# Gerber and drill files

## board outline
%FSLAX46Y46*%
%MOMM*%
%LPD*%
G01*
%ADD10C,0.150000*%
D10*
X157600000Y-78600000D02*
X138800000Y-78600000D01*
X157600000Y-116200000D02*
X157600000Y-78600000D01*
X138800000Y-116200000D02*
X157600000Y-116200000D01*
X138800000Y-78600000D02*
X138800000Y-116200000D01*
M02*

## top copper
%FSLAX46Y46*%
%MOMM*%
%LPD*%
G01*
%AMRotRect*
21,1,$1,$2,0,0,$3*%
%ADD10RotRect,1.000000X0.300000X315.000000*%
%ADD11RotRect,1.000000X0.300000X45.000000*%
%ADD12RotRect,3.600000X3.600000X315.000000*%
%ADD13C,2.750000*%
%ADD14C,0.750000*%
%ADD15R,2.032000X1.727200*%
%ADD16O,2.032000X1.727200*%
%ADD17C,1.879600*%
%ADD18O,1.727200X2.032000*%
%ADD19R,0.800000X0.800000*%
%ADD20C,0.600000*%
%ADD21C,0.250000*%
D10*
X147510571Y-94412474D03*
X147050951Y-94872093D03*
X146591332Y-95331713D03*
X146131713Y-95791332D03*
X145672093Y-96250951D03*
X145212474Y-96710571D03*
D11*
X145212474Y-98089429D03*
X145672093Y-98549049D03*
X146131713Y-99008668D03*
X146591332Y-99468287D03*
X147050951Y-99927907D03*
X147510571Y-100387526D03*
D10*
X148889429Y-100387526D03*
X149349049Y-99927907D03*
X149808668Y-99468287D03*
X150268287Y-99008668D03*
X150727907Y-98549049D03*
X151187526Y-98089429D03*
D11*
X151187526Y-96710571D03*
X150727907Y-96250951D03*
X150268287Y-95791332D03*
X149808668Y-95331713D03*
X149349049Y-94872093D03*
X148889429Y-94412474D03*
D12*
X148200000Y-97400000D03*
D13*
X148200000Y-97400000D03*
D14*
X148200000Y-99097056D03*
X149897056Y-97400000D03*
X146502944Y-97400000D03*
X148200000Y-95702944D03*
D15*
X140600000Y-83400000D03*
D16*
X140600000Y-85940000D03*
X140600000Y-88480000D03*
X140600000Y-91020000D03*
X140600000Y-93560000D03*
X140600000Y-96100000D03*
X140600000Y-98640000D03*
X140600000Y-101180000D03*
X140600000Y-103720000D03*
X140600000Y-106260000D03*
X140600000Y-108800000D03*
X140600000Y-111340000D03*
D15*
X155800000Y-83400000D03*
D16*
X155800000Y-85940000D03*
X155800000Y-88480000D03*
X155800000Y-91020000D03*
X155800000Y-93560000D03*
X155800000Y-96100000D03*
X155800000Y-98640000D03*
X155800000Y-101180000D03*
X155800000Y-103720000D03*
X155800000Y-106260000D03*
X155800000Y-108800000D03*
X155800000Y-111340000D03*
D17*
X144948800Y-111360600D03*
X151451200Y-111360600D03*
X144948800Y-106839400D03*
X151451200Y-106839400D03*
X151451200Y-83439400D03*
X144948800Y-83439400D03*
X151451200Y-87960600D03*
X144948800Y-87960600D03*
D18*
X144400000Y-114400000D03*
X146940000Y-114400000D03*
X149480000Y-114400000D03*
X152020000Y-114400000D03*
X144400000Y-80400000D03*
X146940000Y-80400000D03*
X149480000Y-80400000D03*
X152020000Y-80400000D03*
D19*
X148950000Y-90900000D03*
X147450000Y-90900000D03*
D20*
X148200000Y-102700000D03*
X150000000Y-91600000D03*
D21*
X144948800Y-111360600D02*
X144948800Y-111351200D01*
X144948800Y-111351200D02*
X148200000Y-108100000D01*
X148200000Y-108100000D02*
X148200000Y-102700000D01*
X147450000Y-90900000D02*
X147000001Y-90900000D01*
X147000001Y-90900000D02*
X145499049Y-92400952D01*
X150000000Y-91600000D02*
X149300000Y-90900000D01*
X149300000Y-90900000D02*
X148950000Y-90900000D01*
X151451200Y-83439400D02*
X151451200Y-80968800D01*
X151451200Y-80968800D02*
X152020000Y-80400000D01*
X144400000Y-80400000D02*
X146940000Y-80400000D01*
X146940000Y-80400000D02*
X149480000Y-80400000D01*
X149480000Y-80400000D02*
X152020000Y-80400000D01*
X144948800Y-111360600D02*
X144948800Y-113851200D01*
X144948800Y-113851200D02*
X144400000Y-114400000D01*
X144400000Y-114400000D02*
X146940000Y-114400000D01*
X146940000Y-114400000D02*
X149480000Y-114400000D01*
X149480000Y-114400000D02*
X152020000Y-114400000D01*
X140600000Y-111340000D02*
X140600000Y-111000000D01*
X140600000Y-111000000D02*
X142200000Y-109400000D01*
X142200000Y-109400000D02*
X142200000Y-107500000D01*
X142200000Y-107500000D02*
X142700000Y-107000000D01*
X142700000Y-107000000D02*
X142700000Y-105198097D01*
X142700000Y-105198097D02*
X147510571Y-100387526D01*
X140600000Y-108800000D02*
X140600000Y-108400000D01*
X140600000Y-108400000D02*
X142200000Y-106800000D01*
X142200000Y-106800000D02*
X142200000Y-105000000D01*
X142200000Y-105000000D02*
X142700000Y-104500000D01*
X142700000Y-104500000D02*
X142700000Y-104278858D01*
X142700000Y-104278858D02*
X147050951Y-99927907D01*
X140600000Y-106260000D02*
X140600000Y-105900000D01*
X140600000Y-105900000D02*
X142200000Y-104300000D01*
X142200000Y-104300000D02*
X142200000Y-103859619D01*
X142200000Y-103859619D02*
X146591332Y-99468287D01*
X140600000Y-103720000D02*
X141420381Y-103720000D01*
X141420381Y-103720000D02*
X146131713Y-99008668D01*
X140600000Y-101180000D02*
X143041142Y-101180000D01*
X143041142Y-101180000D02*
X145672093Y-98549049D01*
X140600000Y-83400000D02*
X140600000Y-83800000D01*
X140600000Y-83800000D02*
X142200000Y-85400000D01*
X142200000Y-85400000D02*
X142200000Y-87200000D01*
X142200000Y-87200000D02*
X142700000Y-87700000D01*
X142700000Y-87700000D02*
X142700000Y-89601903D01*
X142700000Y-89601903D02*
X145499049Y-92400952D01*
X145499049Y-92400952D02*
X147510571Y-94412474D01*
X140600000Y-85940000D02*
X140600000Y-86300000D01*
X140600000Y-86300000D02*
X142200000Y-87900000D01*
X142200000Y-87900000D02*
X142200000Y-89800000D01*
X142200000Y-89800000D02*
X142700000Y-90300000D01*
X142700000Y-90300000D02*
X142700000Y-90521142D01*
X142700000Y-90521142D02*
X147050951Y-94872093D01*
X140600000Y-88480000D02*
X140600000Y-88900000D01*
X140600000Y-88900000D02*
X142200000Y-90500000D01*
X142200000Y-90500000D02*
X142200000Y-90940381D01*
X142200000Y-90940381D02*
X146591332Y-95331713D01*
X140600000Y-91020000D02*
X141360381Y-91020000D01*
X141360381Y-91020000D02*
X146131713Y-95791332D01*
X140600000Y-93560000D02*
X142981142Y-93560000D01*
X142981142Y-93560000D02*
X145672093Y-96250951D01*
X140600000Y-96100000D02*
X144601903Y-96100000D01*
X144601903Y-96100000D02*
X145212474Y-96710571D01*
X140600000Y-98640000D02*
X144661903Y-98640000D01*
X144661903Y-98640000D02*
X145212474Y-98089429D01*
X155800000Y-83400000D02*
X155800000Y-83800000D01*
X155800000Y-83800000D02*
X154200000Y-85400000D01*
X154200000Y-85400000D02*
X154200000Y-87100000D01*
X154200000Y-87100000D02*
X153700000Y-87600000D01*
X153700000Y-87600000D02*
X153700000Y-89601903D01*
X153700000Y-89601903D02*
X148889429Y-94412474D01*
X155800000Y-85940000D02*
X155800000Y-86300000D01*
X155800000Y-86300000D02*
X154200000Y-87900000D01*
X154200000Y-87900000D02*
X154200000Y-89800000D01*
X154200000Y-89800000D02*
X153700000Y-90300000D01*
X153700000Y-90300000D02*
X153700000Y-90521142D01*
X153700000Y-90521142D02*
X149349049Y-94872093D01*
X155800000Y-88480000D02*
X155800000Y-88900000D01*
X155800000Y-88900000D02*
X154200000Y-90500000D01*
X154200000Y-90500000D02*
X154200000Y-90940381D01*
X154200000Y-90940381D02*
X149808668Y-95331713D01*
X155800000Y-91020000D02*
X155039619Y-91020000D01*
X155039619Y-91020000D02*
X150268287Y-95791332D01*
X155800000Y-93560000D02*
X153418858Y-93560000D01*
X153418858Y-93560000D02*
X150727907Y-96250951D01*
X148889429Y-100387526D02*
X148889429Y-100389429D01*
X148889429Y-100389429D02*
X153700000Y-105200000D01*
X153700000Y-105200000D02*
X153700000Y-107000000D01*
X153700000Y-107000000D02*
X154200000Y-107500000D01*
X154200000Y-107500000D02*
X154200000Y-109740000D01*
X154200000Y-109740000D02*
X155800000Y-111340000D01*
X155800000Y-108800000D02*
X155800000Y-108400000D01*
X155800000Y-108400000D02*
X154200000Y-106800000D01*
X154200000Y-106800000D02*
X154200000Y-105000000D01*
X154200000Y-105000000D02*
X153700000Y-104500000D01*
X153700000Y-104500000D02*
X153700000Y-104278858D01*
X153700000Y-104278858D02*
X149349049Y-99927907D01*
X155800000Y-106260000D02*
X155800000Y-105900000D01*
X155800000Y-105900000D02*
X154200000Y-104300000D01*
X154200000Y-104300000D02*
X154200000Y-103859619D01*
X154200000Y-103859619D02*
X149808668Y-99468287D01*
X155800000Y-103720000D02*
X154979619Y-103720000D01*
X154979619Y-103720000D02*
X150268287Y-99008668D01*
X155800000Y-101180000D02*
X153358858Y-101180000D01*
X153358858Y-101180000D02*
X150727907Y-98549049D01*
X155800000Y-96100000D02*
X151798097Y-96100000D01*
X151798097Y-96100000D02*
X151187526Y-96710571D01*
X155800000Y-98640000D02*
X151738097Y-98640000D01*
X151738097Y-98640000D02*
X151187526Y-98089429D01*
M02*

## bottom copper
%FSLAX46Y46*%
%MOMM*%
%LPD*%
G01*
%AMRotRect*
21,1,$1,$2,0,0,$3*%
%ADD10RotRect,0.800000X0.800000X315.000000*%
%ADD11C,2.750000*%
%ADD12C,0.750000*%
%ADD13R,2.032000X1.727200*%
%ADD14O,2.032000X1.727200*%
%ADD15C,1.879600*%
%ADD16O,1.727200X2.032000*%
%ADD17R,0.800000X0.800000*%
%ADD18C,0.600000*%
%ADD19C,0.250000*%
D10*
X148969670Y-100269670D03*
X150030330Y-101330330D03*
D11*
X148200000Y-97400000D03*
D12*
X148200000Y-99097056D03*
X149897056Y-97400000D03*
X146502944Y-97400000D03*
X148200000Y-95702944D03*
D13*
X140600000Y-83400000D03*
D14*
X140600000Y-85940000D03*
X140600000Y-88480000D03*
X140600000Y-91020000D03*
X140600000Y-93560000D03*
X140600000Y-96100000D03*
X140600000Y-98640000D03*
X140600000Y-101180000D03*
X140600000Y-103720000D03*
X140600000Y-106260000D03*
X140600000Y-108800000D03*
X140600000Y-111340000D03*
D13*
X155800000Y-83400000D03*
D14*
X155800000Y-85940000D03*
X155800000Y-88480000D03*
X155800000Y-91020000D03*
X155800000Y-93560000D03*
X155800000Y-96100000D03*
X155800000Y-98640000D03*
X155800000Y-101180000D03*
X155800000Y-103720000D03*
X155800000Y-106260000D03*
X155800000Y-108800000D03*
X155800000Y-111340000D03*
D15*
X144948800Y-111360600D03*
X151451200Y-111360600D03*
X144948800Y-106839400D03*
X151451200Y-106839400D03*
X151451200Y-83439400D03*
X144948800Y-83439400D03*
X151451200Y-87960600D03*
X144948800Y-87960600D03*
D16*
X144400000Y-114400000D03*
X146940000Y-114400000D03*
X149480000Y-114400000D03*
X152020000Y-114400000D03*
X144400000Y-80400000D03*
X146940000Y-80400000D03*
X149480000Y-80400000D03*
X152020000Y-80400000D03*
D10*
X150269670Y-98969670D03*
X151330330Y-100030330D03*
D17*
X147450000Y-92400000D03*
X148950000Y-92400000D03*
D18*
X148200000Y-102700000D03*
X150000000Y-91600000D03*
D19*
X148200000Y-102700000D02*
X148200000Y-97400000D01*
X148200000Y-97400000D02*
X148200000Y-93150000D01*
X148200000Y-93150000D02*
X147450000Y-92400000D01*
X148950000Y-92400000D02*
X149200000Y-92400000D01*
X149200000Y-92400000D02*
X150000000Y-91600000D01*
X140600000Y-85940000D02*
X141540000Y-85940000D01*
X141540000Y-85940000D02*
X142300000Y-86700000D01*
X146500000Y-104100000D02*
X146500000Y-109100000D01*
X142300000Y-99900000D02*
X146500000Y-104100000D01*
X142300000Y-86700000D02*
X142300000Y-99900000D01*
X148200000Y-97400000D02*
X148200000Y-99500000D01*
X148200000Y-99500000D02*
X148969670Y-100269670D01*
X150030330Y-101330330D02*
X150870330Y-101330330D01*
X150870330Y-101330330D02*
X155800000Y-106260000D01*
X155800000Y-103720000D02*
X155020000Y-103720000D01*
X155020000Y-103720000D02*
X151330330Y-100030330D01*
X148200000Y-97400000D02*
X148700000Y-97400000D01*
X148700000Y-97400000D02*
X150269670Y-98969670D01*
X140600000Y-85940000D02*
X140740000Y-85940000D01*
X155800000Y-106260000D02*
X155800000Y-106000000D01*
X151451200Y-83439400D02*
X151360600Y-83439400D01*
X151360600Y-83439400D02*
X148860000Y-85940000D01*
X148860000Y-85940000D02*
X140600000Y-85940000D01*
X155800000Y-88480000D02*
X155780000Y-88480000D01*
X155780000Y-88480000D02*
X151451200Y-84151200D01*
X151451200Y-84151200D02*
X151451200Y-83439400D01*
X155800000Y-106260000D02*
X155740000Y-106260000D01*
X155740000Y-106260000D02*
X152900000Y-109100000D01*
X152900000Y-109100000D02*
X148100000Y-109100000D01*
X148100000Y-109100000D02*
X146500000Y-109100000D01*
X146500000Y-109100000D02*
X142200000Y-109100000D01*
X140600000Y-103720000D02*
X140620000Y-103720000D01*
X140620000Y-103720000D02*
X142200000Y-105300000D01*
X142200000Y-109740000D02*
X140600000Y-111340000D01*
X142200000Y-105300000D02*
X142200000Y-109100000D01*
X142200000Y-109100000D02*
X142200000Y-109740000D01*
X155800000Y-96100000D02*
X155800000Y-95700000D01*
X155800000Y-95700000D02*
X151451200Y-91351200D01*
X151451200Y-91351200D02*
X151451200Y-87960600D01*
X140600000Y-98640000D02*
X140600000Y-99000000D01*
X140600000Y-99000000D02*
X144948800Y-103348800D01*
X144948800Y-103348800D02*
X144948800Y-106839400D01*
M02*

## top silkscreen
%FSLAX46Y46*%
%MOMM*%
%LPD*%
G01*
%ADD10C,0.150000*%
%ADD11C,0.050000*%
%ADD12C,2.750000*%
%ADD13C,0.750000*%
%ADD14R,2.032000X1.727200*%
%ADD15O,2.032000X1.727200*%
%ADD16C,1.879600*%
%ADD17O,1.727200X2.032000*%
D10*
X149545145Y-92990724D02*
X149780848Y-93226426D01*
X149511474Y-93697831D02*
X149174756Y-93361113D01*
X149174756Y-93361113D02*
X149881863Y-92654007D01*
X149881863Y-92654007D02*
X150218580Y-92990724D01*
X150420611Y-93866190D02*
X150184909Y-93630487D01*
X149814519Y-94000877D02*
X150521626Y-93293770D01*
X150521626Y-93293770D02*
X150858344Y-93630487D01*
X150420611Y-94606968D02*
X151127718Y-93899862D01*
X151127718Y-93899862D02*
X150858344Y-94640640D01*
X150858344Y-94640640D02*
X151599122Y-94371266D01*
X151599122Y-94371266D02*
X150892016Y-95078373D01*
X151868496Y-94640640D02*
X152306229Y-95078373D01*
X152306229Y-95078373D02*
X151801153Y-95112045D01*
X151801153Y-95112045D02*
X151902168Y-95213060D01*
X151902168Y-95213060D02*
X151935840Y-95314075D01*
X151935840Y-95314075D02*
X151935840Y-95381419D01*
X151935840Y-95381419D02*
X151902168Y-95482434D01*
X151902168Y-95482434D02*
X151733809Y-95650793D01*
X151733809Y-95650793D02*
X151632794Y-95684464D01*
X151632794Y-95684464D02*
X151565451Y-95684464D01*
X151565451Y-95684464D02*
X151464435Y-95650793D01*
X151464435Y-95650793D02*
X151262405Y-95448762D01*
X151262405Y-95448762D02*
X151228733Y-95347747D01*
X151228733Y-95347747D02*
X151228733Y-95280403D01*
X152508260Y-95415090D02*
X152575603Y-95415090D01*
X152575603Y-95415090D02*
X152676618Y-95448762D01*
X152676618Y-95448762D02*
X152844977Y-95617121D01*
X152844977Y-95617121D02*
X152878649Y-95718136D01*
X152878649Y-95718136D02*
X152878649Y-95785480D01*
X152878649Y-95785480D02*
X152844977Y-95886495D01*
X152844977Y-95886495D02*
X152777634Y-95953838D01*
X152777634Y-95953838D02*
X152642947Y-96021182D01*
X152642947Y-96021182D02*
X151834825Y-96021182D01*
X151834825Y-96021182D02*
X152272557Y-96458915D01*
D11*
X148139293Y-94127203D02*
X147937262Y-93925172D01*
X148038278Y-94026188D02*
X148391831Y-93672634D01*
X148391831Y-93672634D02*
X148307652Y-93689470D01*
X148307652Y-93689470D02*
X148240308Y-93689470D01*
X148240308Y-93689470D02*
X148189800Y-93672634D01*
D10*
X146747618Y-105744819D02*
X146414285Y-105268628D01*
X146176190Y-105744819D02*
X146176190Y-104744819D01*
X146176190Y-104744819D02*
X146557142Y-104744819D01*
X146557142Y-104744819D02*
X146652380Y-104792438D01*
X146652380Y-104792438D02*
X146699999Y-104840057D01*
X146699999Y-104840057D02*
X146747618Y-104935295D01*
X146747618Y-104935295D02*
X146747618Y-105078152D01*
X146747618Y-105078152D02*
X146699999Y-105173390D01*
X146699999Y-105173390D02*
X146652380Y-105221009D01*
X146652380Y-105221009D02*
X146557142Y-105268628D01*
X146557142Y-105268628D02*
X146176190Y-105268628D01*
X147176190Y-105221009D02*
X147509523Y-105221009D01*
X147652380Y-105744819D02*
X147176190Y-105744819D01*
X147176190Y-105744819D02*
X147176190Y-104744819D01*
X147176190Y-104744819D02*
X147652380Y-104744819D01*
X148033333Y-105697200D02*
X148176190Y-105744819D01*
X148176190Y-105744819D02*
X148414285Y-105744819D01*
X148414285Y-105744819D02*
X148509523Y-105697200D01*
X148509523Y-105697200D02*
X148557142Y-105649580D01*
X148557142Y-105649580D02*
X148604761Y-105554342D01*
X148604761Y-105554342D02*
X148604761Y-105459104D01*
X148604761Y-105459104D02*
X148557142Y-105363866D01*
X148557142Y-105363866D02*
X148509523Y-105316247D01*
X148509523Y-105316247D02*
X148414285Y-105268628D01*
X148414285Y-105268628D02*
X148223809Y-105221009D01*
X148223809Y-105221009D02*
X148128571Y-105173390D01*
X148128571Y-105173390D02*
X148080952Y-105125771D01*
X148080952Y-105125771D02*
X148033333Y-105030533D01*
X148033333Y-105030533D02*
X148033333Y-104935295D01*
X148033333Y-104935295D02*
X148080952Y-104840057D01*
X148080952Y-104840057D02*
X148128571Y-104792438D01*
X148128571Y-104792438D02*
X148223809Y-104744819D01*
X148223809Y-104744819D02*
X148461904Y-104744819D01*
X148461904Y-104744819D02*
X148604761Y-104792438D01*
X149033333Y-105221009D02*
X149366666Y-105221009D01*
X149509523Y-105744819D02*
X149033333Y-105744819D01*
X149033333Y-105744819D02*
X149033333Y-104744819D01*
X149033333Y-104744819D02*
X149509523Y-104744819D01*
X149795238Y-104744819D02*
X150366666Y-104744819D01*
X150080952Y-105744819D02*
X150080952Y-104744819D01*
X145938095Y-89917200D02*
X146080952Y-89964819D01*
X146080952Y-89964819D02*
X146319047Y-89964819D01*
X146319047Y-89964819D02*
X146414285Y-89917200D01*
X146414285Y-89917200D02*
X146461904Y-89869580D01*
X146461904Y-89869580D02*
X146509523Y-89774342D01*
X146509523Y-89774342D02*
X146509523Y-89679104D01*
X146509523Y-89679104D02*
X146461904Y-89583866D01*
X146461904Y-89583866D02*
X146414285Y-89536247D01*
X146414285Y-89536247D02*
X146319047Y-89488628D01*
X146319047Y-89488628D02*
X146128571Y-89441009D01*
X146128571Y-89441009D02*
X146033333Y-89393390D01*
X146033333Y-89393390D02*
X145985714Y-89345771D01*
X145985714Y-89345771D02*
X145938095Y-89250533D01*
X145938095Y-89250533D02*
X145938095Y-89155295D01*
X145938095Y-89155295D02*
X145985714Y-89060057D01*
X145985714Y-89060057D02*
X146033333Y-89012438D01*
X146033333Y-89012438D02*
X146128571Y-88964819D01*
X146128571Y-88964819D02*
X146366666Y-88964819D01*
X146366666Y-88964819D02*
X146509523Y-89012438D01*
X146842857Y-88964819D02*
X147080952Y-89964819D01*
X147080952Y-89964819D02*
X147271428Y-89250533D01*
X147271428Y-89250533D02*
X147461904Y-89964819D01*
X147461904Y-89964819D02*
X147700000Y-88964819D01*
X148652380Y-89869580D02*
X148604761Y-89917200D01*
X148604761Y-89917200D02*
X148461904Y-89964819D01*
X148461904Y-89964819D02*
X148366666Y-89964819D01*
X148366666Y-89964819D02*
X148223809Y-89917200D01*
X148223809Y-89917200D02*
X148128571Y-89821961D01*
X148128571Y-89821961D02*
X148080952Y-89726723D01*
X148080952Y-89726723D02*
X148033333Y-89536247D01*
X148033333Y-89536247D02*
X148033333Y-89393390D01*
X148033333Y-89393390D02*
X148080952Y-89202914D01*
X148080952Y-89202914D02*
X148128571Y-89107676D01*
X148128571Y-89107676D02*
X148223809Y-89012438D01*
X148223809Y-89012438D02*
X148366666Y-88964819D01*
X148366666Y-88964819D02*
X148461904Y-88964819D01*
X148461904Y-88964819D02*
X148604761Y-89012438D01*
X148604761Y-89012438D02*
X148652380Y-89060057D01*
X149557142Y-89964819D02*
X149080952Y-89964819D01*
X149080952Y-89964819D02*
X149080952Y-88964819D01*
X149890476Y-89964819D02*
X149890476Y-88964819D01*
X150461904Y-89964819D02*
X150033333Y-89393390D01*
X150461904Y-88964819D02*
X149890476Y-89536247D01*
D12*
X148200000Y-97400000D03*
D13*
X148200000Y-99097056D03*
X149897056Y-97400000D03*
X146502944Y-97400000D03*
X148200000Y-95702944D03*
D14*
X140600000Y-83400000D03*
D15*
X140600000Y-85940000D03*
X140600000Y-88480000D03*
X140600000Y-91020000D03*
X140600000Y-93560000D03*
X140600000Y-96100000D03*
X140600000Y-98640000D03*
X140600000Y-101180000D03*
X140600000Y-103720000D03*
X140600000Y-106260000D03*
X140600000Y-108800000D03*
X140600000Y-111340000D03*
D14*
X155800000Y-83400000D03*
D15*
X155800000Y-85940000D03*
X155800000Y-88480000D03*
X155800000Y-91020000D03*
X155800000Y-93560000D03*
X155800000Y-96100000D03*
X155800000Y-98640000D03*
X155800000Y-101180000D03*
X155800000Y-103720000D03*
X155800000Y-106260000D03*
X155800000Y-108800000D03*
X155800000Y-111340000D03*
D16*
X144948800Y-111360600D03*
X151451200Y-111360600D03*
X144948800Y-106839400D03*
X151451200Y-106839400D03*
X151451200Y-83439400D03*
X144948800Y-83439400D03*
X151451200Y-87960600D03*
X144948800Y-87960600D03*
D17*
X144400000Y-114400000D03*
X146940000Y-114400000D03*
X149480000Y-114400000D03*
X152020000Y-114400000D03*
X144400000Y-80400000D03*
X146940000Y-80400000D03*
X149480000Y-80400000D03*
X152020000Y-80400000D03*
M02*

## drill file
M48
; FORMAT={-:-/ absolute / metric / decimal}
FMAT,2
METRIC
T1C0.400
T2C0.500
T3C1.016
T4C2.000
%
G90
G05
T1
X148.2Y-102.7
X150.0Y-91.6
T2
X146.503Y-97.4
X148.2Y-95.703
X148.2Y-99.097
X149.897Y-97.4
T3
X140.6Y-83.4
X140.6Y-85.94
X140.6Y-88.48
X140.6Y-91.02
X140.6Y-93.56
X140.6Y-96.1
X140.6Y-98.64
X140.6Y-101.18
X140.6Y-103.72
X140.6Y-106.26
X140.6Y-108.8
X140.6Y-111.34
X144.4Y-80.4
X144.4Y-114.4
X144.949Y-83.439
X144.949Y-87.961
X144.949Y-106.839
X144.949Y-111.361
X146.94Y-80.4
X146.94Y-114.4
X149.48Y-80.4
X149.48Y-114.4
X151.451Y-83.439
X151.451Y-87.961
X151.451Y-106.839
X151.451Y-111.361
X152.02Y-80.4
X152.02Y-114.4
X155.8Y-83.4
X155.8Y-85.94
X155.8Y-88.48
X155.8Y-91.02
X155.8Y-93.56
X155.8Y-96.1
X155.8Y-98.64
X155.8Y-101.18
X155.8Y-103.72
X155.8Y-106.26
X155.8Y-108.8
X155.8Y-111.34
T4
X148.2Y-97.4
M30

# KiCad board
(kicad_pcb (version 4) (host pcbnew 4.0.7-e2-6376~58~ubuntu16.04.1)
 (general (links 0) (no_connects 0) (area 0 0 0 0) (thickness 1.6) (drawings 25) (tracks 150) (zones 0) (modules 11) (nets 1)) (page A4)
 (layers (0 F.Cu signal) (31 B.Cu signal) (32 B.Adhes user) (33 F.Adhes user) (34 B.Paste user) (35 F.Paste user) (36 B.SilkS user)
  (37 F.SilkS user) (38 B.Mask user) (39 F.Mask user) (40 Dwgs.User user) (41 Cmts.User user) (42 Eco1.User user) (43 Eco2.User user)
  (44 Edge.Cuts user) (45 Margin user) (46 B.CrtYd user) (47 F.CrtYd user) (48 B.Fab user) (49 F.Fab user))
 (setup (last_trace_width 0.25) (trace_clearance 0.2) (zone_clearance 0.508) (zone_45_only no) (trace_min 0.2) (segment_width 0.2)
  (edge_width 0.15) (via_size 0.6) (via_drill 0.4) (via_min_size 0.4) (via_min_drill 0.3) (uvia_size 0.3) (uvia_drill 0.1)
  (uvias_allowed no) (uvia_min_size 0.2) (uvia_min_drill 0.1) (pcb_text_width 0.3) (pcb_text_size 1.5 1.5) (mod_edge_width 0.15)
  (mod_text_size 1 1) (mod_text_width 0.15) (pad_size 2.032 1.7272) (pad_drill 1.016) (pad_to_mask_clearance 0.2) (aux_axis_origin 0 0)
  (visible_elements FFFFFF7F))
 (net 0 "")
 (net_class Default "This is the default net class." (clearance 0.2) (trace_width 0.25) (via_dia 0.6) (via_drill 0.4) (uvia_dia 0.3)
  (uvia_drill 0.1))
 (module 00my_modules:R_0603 (layer B.Cu) (at 149.5 100.8 315)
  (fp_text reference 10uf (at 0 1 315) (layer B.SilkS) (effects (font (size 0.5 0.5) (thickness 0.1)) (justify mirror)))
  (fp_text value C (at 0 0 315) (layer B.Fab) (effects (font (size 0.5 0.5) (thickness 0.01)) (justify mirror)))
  (pad 1 smd rect (at -0.75 0 315) (size 0.8 0.8) (layers B.Cu B.Paste B.Mask))
  (pad 2 smd rect (at 0.75 0 315) (size 0.8 0.8) (layers B.Cu B.Paste B.Mask)))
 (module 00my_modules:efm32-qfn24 (layer F.Cu) (at 148.2 97.4 315)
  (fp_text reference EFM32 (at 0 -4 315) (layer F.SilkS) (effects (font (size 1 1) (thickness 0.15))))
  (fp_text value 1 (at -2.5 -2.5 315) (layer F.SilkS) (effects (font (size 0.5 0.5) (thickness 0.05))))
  (pad 1 smd rect (at -2.6 -1.625 315) (size 1 0.3) (layers F.Cu F.Paste F.Mask))
  (pad 2 smd rect (at -2.6 -0.975 315) (size 1 0.3) (layers F.Cu F.Paste F.Mask))
  (pad 3 smd rect (at -2.6 -0.325 315) (size 1 0.3) (layers F.Cu F.Paste F.Mask))
  (pad 4 smd rect (at -2.6 0.325 315) (size 1 0.3) (layers F.Cu F.Paste F.Mask))
  (pad 5 smd rect (at -2.6 0.975 315) (size 1 0.3) (layers F.Cu F.Paste F.Mask))
  (pad 6 smd rect (at -2.6 1.625 315) (size 1 0.3) (layers F.Cu F.Paste F.Mask))
  (pad 7 smd rect (at -1.625 2.6 45) (size 1 0.3) (layers F.Cu F.Paste F.Mask))
  (pad 8 smd rect (at -0.975 2.6 45) (size 1 0.3) (layers F.Cu F.Paste F.Mask))
  (pad 9 smd rect (at -0.325 2.6 45) (size 1 0.3) (layers F.Cu F.Paste F.Mask))
  (pad 10 smd rect (at 0.325 2.6 45) (size 1 0.3) (layers F.Cu F.Paste F.Mask))
  (pad 11 smd rect (at 0.975 2.6 45) (size 1 0.3) (layers F.Cu F.Paste F.Mask))
  (pad 12 smd rect (at 1.625 2.6 45) (size 1 0.3) (layers F.Cu F.Paste F.Mask))
  (pad 13 smd rect (at 2.6 1.625 315) (size 1 0.3) (layers F.Cu F.Paste F.Mask))
  (pad 14 smd rect (at 2.6 0.975 315) (size 1 0.3) (layers F.Cu F.Paste F.Mask))
  (pad 15 smd rect (at 2.6 0.325 315) (size 1 0.3) (layers F.Cu F.Paste F.Mask))
  (pad 16 smd rect (at 2.6 -0.325 315) (size 1 0.3) (layers F.Cu F.Paste F.Mask))
  (pad 17 smd rect (at 2.6 -0.975 315) (size 1 0.3) (layers F.Cu F.Paste F.Mask))
  (pad 18 smd rect (at 2.6 -1.625 315) (size 1 0.3) (layers F.Cu F.Paste F.Mask))
  (pad 19 smd rect (at 1.625 -2.6 45) (size 1 0.3) (layers F.Cu F.Paste F.Mask))
  (pad 20 smd rect (at 0.975 -2.6 45) (size 1 0.3) (layers F.Cu F.Paste F.Mask))
  (pad 21 smd rect (at 0.325 -2.6 45) (size 1 0.3) (layers F.Cu F.Paste F.Mask))
  (pad 22 smd rect (at -0.325 -2.6 45) (size 1 0.3) (layers F.Cu F.Paste F.Mask))
  (pad 23 smd rect (at -0.975 -2.6 45) (size 1 0.3) (layers F.Cu F.Paste F.Mask))
  (pad 24 smd rect (at -1.625 -2.6 45) (size 1 0.3) (layers F.Cu F.Paste F.Mask))
  (pad 25 smd rect (at 0 0 315) (size 3.6 3.6) (layers F.Cu F.Paste F.Mask))
  (pad "" thru_hole circle (at 0 0 315) (size 2.75 2.75) (drill 2) (layers *.Cu *.Mask F.SilkS))
  (pad "" thru_hole circle (at 1.2 1.2 315) (size 0.75 0.75) (drill 0.5) (layers *.Cu *.Mask F.SilkS))
  (pad "" thru_hole circle (at 1.2 -1.2 315) (size 0.75 0.75) (drill 0.5) (layers *.Cu *.Mask F.SilkS))
  (pad "" thru_hole circle (at -1.2 1.2 315) (size 0.75 0.75) (drill 0.5) (layers *.Cu *.Mask F.SilkS))
  (pad "" thru_hole circle (at -1.2 -1.2 315) (size 0.75 0.75) (drill 0.5) (layers *.Cu *.Mask F.SilkS)))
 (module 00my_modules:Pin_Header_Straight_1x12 (layer F.Cu) (at 140.6 83.4)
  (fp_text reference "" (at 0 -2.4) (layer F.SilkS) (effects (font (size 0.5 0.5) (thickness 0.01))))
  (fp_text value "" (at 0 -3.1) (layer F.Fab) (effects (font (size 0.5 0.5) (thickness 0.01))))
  (pad 1 thru_hole rect (at 0 0) (size 2.032 1.7272) (drill 1.016) (layers *.Cu *.Mask F.SilkS))
  (pad 2 thru_hole oval (at 0 2.54) (size 2.032 1.7272) (drill 1.016) (layers *.Cu *.Mask F.SilkS))
  (pad 3 thru_hole oval (at 0 5.08) (size 2.032 1.7272) (drill 1.016) (layers *.Cu *.Mask F.SilkS))
  (pad 4 thru_hole oval (at 0 7.62) (size 2.032 1.7272) (drill 1.016) (layers *.Cu *.Mask F.SilkS))
  (pad 5 thru_hole oval (at 0 10.16) (size 2.032 1.7272) (drill 1.016) (layers *.Cu *.Mask F.SilkS))
  (pad 6 thru_hole oval (at 0 12.7) (size 2.032 1.7272) (drill 1.016) (layers *.Cu *.Mask F.SilkS))
  (pad 7 thru_hole oval (at 0 15.24) (size 2.032 1.7272) (drill 1.016) (layers *.Cu *.Mask F.SilkS))
  (pad 8 thru_hole oval (at 0 17.78) (size 2.032 1.7272) (drill 1.016) (layers *.Cu *.Mask F.SilkS))
  (pad 9 thru_hole oval (at 0 20.32) (size 2.032 1.7272) (drill 1.016) (layers *.Cu *.Mask F.SilkS))
  (pad 10 thru_hole oval (at 0 22.86) (size 2.032 1.7272) (drill 1.016) (layers *.Cu *.Mask F.SilkS))
  (pad 11 thru_hole oval (at 0 25.4) (size 2.032 1.7272) (drill 1.016) (layers *.Cu *.Mask F.SilkS))
  (pad 12 thru_hole oval (at 0 27.94) (size 2.032 1.7272) (drill 1.016) (layers *.Cu *.Mask F.SilkS)))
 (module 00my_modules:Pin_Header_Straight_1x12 (layer F.Cu) (at 155.8 83.4)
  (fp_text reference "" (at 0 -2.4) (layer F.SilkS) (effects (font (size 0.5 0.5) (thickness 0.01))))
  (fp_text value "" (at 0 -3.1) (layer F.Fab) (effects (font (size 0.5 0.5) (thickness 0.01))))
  (pad 24 thru_hole rect (at 0 0) (size 2.032 1.7272) (drill 1.016) (layers *.Cu *.Mask F.SilkS))
  (pad 23 thru_hole oval (at 0 2.54) (size 2.032 1.7272) (drill 1.016) (layers *.Cu *.Mask F.SilkS))
  (pad 22 thru_hole oval (at 0 5.08) (size 2.032 1.7272) (drill 1.016) (layers *.Cu *.Mask F.SilkS))
  (pad 21 thru_hole oval (at 0 7.62) (size 2.032 1.7272) (drill 1.016) (layers *.Cu *.Mask F.SilkS))
  (pad 20 thru_hole oval (at 0 10.16) (size 2.032 1.7272) (drill 1.016) (layers *.Cu *.Mask F.SilkS))
  (pad 19 thru_hole oval (at 0 12.7) (size 2.032 1.7272) (drill 1.016) (layers *.Cu *.Mask F.SilkS))
  (pad 18 thru_hole oval (at 0 15.24) (size 2.032 1.7272) (drill 1.016) (layers *.Cu *.Mask F.SilkS))
  (pad 17 thru_hole oval (at 0 17.78) (size 2.032 1.7272) (drill 1.016) (layers *.Cu *.Mask F.SilkS))
  (pad 16 thru_hole oval (at 0 20.32) (size 2.032 1.7272) (drill 1.016) (layers *.Cu *.Mask F.SilkS))
  (pad 15 thru_hole oval (at 0 22.86) (size 2.032 1.7272) (drill 1.016) (layers *.Cu *.Mask F.SilkS))
  (pad 14 thru_hole oval (at 0 25.4) (size 2.032 1.7272) (drill 1.016) (layers *.Cu *.Mask F.SilkS))
  (pad 13 thru_hole oval (at 0 27.94) (size 2.032 1.7272) (drill 1.016) (layers *.Cu *.Mask F.SilkS)))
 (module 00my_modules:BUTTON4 (layer F.Cu) (at 148.2 109.1)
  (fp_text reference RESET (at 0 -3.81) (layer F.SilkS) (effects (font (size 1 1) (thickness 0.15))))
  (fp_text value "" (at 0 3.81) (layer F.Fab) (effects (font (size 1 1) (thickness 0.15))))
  (pad 1 thru_hole circle (at -3.2512 2.2606) (size 1.8796 1.8796) (drill 1.016) (layers *.Cu *.Mask F.SilkS))
  (pad 2 thru_hole circle (at 3.2512 2.2606) (size 1.8796 1.8796) (drill 1.016) (layers *.Cu *.Mask F.SilkS))
  (pad 3 thru_hole circle (at -3.2512 -2.2606) (size 1.8796 1.8796) (drill 1.016) (layers *.Cu *.Mask F.SilkS))
  (pad 4 thru_hole circle (at 3.2512 -2.2606) (size 1.8796 1.8796) (drill 1.016) (layers *.Cu *.Mask F.SilkS)))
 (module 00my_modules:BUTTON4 (layer F.Cu) (at 148.2 85.7 180)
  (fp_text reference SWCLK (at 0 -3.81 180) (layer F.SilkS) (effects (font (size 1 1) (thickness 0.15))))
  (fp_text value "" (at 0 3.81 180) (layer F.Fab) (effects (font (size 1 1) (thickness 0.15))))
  (pad 1 thru_hole circle (at -3.2512 2.2606 180) (size 1.8796 1.8796) (drill 1.016) (layers *.Cu *.Mask F.SilkS))
  (pad 2 thru_hole circle (at 3.2512 2.2606 180) (size 1.8796 1.8796) (drill 1.016) (layers *.Cu *.Mask F.SilkS))
  (pad 3 thru_hole circle (at -3.2512 -2.2606 180) (size 1.8796 1.8796) (drill 1.016) (layers *.Cu *.Mask F.SilkS))
  (pad 4 thru_hole circle (at 3.2512 -2.2606 180) (size 1.8796 1.8796) (drill 1.016) (layers *.Cu *.Mask F.SilkS)))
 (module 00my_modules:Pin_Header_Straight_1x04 (layer F.Cu) (at 144.4 114.4 90)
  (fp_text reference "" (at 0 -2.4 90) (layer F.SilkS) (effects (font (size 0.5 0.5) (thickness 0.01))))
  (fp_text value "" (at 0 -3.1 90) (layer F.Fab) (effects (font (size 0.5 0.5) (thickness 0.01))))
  (pad 1 thru_hole oval (at 0 0 90) (size 2.032 1.7272) (drill 1.016) (layers *.Cu *.Mask F.SilkS))
  (pad 2 thru_hole oval (at 0 2.54 90) (size 2.032 1.7272) (drill 1.016) (layers *.Cu *.Mask F.SilkS))
  (pad 3 thru_hole oval (at 0 5.08 90) (size 2.032 1.7272) (drill 1.016) (layers *.Cu *.Mask F.SilkS))
  (pad 4 thru_hole oval (at 0 7.62 90) (size 2.032 1.7272) (drill 1.016) (layers *.Cu *.Mask F.SilkS)))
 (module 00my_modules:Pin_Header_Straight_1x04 (layer F.Cu) (at 144.4 80.4 90)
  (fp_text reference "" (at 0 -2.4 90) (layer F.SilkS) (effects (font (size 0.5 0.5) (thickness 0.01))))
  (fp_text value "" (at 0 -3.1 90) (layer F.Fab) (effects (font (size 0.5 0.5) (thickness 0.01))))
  (pad 1 thru_hole oval (at 0 0 90) (size 2.032 1.7272) (drill 1.016) (layers *.Cu *.Mask F.SilkS))
  (pad 2 thru_hole oval (at 0 2.54 90) (size 2.032 1.7272) (drill 1.016) (layers *.Cu *.Mask F.SilkS))
  (pad 3 thru_hole oval (at 0 5.08 90) (size 2.032 1.7272) (drill 1.016) (layers *.Cu *.Mask F.SilkS))
  (pad 4 thru_hole oval (at 0 7.62 90) (size 2.032 1.7272) (drill 1.016) (layers *.Cu *.Mask F.SilkS)))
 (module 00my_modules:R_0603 (layer B.Cu) (at 150.8 99.5 315)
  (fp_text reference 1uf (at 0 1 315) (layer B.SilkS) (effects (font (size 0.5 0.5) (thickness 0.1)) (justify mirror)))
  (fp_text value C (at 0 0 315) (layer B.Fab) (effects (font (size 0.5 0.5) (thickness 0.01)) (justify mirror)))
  (pad 1 smd rect (at -0.75 0 315) (size 0.8 0.8) (layers B.Cu B.Paste B.Mask))
  (pad 2 smd rect (at 0.75 0 315) (size 0.8 0.8) (layers B.Cu B.Paste B.Mask)))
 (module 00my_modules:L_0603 (layer F.Cu) (at 148.2 90.9 180)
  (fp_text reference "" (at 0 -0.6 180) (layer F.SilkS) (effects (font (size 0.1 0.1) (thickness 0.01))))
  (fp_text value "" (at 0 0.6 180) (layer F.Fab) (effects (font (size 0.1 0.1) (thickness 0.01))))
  (pad 1 smd rect (at -0.75 0 180) (size 0.8 0.8) (layers F.Cu F.Paste F.Mask))
  (pad 2 smd rect (at 0.75 0 180) (size 0.8 0.8) (layers F.Cu F.Paste F.Mask)))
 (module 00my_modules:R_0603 (layer B.Cu) (at 148.2 92.4)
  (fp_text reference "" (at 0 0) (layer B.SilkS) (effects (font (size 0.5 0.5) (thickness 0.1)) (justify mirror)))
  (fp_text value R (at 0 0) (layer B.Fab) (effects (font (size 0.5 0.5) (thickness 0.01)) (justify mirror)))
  (pad 1 smd rect (at -0.75 0) (size 0.8 0.8) (layers B.Cu B.Paste B.Mask))
  (pad 2 smd rect (at 0.75 0) (size 0.8 0.8) (layers B.Cu B.Paste B.Mask)))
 (gr_line (start 157.6 78.6) (end 138.8 78.6) (angle 90) (layer Edge.Cuts) (width 0.15))
 (gr_line (start 157.6 116.2) (end 157.6 78.6) (angle 90) (layer Edge.Cuts) (width 0.15))
 (gr_line (start 138.8 116.2) (end 157.6 116.2) (angle 90) (layer Edge.Cuts) (width 0.15))
 (gr_line (start 138.8 78.6) (end 138.8 116.2) (angle 90) (layer Edge.Cuts) (width 0.15))
 (segment (start 144.9488 111.3606) (end 144.9488 111.3512) (width 0.25) (layer F.Cu) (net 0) (status C00000))
 (segment (start 144.9488 111.3512) (end 148.2 108.1) (width 0.25) (layer F.Cu) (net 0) (status 400000))
 (segment (start 148.2 102.7) (end 148.2 97.4) (width 0.25) (layer B.Cu) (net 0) (status 800000))
 (via (at 148.2 102.7) (size 0.6) (drill 0.4) (layers F.Cu B.Cu) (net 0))
 (segment (start 148.2 108.1) (end 148.2 102.7) (width 0.25) (layer F.Cu) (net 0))
 (segment (start 148.2 97.4) (end 148.2 93.15) (width 0.25) (layer B.Cu) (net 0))
 (segment (start 148.2 93.15) (end 147.45 92.4) (width 0.25) (layer B.Cu) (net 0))
 (segment (start 147.45 90.9) (end 147.000001 90.9) (width 0.25) (layer F.Cu) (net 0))
 (segment (start 147.000001 90.9) (end 145.499049 92.400952) (width 0.25) (layer F.Cu) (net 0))
 (segment (start 148.95 92.4) (end 149.2 92.4) (width 0.25) (layer B.Cu) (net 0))
 (segment (start 149.2 92.4) (end 150 91.6) (width 0.25) (layer B.Cu) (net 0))
 (via (at 150 91.6) (size 0.6) (drill 0.4) (layers F.Cu B.Cu) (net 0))
 (segment (start 150 91.6) (end 149.3 90.9) (width 0.25) (layer F.Cu) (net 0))
 (segment (start 149.3 90.9) (end 148.95 90.9) (width 0.25) (layer F.Cu) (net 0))
 (segment (start 140.6 85.94) (end 141.54 85.94) (width 0.25) (layer B.Cu) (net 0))
 (segment (start 141.54 85.94) (end 142.3 86.7) (width 0.25) (layer B.Cu) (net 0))
 (segment (start 146.5 104.1) (end 146.5 109.1) (width 0.25) (layer B.Cu) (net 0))
 (segment (start 142.3 99.9) (end 146.5 104.1) (width 0.25) (layer B.Cu) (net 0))
 (segment (start 142.3 86.7) (end 142.3 99.9) (width 0.25) (layer B.Cu) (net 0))
 (segment (start 148.2 97.4) (end 148.2 99.5) (width 0.25) (layer B.Cu) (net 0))
 (segment (start 148.2 99.5) (end 148.96967 100.26967) (width 0.25) (layer B.Cu) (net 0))
 (segment (start 150.03033 101.33033) (end 150.87033 101.33033) (width 0.25) (layer B.Cu) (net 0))
 (segment (start 150.87033 101.33033) (end 155.8 106.26) (width 0.25) (layer B.Cu) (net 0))
 (segment (start 155.8 103.72) (end 155.02 103.72) (width 0.25) (layer B.Cu) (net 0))
 (segment (start 155.02 103.72) (end 151.33033 100.03033) (width 0.25) (layer B.Cu) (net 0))
 (segment (start 148.2 97.4) (end 148.7 97.4) (width 0.25) (layer B.Cu) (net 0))
 (segment (start 148.7 97.4) (end 150.26967 98.96967) (width 0.25) (layer B.Cu) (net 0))
 (segment (start 140.6 85.94) (end 140.74 85.94) (width 0.25) (layer B.Cu) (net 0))
 (segment (start 155.8 106.26) (end 155.8 106) (width 0.25) (layer B.Cu) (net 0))
 (segment (start 151.4512 83.4394) (end 151.3606 83.4394) (width 0.25) (layer B.Cu) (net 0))
 (segment (start 151.3606 83.4394) (end 148.86 85.94) (width 0.25) (layer B.Cu) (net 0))
 (segment (start 148.86 85.94) (end 140.6 85.94) (width 0.25) (layer B.Cu) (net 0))
 (segment (start 155.8 88.48) (end 155.78 88.48) (width 0.25) (layer B.Cu) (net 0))
 (segment (start 155.78 88.48) (end 151.4512 84.1512) (width 0.25) (layer B.Cu) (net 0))
 (segment (start 151.4512 84.1512) (end 151.4512 83.4394) (width 0.25) (layer B.Cu) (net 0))
 (segment (start 155.8 106.26) (end 155.74 106.26) (width 0.25) (layer B.Cu) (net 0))
 (segment (start 155.74 106.26) (end 152.9 109.1) (width 0.25) (layer B.Cu) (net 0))
 (segment (start 152.9 109.1) (end 148.1 109.1) (width 0.25) (layer B.Cu) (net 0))
 (segment (start 148.1 109.1) (end 146.5 109.1) (width 0.25) (layer B.Cu) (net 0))
 (segment (start 146.5 109.1) (end 142.2 109.1) (width 0.25) (layer B.Cu) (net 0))
 (segment (start 140.6 103.72) (end 140.62 103.72) (width 0.25) (layer B.Cu) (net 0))
 (segment (start 140.62 103.72) (end 142.2 105.3) (width 0.25) (layer B.Cu) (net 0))
 (segment (start 142.2 109.74) (end 140.6 111.34) (width 0.25) (layer B.Cu) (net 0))
 (segment (start 142.2 105.3) (end 142.2 109.1) (width 0.25) (layer B.Cu) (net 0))
 (segment (start 142.2 109.1) (end 142.2 109.74) (width 0.25) (layer B.Cu) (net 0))
 (segment (start 151.4512 83.4394) (end 151.4512 80.9688) (width 0.25) (layer F.Cu) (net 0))
 (segment (start 151.4512 80.9688) (end 152.02 80.4) (width 0.25) (layer F.Cu) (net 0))
 (segment (start 155.8 96.1) (end 155.8 95.7) (width 0.25) (layer B.Cu) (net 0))
 (segment (start 155.8 95.7) (end 151.4512 91.3512) (width 0.25) (layer B.Cu) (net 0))
 (segment (start 151.4512 91.3512) (end 151.4512 87.9606) (width 0.25) (layer B.Cu) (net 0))
 (segment (start 144.4 80.4) (end 146.94 80.4) (width 0.25) (layer F.Cu) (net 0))
 (segment (start 146.94 80.4) (end 149.48 80.4) (width 0.25) (layer F.Cu) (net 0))
 (segment (start 149.48 80.4) (end 152.02 80.4) (width 0.25) (layer F.Cu) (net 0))
 (segment (start 144.9488 111.3606) (end 144.9488 113.8512) (width 0.25) (layer F.Cu) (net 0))
 (segment (start 144.9488 113.8512) (end 144.4 114.4) (width 0.25) (layer F.Cu) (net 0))
 (segment (start 144.4 114.4) (end 146.94 114.4) (width 0.25) (layer F.Cu) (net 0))
 (segment (start 146.94 114.4) (end 149.48 114.4) (width 0.25) (layer F.Cu) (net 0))
 (segment (start 149.48 114.4) (end 152.02 114.4) (width 0.25) (layer F.Cu) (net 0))
 (segment (start 140.6 98.64) (end 140.6 99) (width 0.25) (layer B.Cu) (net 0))
 (segment (start 140.6 99) (end 144.9488 103.3488) (width 0.25) (layer B.Cu) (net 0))
 (segment (start 144.9488 103.3488) (end 144.9488 106.8394) (width 0.25) (layer B.Cu) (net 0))
 (segment (start 140.6 111.34) (end 140.6 111) (width 0.25) (layer F.Cu) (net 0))
 (segment (start 140.6 111) (end 142.2 109.4) (width 0.25) (layer F.Cu) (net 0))
 (segment (start 142.2 109.4) (end 142.2 107.5) (width 0.25) (layer F.Cu) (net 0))
 (segment (start 142.2 107.5) (end 142.7 107) (width 0.25) (layer F.Cu) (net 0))
 (segment (start 142.7 107) (end 142.7 105.198097) (width 0.25) (layer F.Cu) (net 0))
 (segment (start 142.7 105.198097) (end 147.510571 100.387526) (width 0.25) (layer F.Cu) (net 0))
 (segment (start 140.6 108.8) (end 140.6 108.4) (width 0.25) (layer F.Cu) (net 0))
 (segment (start 140.6 108.4) (end 142.2 106.8) (width 0.25) (layer F.Cu) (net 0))
 (segment (start 142.2 106.8) (end 142.2 105) (width 0.25) (layer F.Cu) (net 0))
 (segment (start 142.2 105) (end 142.7 104.5) (width 0.25) (layer F.Cu) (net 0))
 (segment (start 142.7 104.5) (end 142.7 104.278858) (width 0.25) (layer F.Cu) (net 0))
 (segment (start 142.7 104.278858) (end 147.050951 99.927907) (width 0.25) (layer F.Cu) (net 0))
 (segment (start 140.6 106.26) (end 140.6 105.9) (width 0.25) (layer F.Cu) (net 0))
 (segment (start 140.6 105.9) (end 142.2 104.3) (width 0.25) (layer F.Cu) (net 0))
 (segment (start 142.2 104.3) (end 142.2 103.859619) (width 0.25) (layer F.Cu) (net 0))
 (segment (start 142.2 103.859619) (end 146.591332 99.468287) (width 0.25) (layer F.Cu) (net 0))
 (segment (start 140.6 103.72) (end 141.420381 103.72) (width 0.25) (layer F.Cu) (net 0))
 (segment (start 141.420381 103.72) (end 146.131713 99.008668) (width 0.25) (layer F.Cu) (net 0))
 (segment (start 140.6 101.18) (end 143.041142 101.18) (width 0.25) (layer F.Cu) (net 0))
 (segment (start 143.041142 101.18) (end 145.672093 98.549049) (width 0.25) (layer F.Cu) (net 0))
 (segment (start 140.6 83.4) (end 140.6 83.8) (width 0.25) (layer F.Cu) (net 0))
 (segment (start 140.6 83.8) (end 142.2 85.4) (width 0.25) (layer F.Cu) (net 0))
 (segment (start 142.2 85.4) (end 142.2 87.2) (width 0.25) (layer F.Cu) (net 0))
 (segment (start 142.2 87.2) (end 142.7 87.7) (width 0.25) (layer F.Cu) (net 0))
 (segment (start 142.7 87.7) (end 142.7 89.601903) (width 0.25) (layer F.Cu) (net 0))
 (segment (start 142.7 89.601903) (end 145.499049 92.400952) (width 0.25) (layer F.Cu) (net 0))
 (segment (start 145.499049 92.400952) (end 147.510571 94.412474) (width 0.25) (layer F.Cu) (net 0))
 (segment (start 140.6 85.94) (end 140.6 86.3) (width 0.25) (layer F.Cu) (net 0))
 (segment (start 140.6 86.3) (end 142.2 87.9) (width 0.25) (layer F.Cu) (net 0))
 (segment (start 142.2 87.9) (end 142.2 89.8) (width 0.25) (layer F.Cu) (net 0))
 (segment (start 142.2 89.8) (end 142.7 90.3) (width 0.25) (layer F.Cu) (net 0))
 (segment (start 142.7 90.3) (end 142.7 90.521142) (width 0.25) (layer F.Cu) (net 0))
 (segment (start 142.7 90.521142) (end 147.050951 94.872093) (width 0.25) (layer F.Cu) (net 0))
 (segment (start 140.6 88.48) (end 140.6 88.9) (width 0.25) (layer F.Cu) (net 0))
 (segment (start 140.6 88.9) (end 142.2 90.5) (width 0.25) (layer F.Cu) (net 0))
 (segment (start 142.2 90.5) (end 142.2 90.940381) (width 0.25) (layer F.Cu) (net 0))
 (segment (start 142.2 90.940381) (end 146.591332 95.331713) (width 0.25) (layer F.Cu) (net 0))
 (segment (start 140.6 91.02) (end 141.360381 91.02) (width 0.25) (layer F.Cu) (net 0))
 (segment (start 141.360381 91.02) (end 146.131713 95.791332) (width 0.25) (layer F.Cu) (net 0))
 (segment (start 140.6 93.56) (end 142.981142 93.56) (width 0.25) (layer F.Cu) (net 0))
 (segment (start 142.981142 93.56) (end 145.672093 96.250951) (width 0.25) (layer F.Cu) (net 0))
 (segment (start 140.6 96.1) (end 144.601903 96.1) (width 0.25) (layer F.Cu) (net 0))
 (segment (start 144.601903 96.1) (end 145.212474 96.710571) (width 0.25) (layer F.Cu) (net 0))
 (segment (start 140.6 98.64) (end 144.661903 98.64) (width 0.25) (layer F.Cu) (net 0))
 (segment (start 144.661903 98.64) (end 145.212474 98.089429) (width 0.25) (layer F.Cu) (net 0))
 (segment (start 155.8 83.4) (end 155.8 83.8) (width 0.25) (layer F.Cu) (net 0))
 (segment (start 155.8 83.8) (end 154.2 85.4) (width 0.25) (layer F.Cu) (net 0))
 (segment (start 154.2 85.4) (end 154.2 87.1) (width 0.25) (layer F.Cu) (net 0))
 (segment (start 154.2 87.1) (end 153.7 87.6) (width 0.25) (layer F.Cu) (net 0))
 (segment (start 153.7 87.6) (end 153.7 89.601903) (width 0.25) (layer F.Cu) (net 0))
 (segment (start 153.7 89.601903) (end 148.889429 94.412474) (width 0.25) (layer F.Cu) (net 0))
 (segment (start 155.8 85.94) (end 155.8 86.3) (width 0.25) (layer F.Cu) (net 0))
 (segment (start 155.8 86.3) (end 154.2 87.9) (width 0.25) (layer F.Cu) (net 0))
 (segment (start 154.2 87.9) (end 154.2 89.8) (width 0.25) (layer F.Cu) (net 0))
 (segment (start 154.2 89.8) (end 153.7 90.3) (width 0.25) (layer F.Cu) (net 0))
 (segment (start 153.7 90.3) (end 153.7 90.521142) (width 0.25) (layer F.Cu) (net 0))
 (segment (start 153.7 90.521142) (end 149.349049 94.872093) (width 0.25) (layer F.Cu) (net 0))
 (segment (start 155.8 88.48) (end 155.8 88.9) (width 0.25) (layer F.Cu) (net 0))
 (segment (start 155.8 88.9) (end 154.2 90.5) (width 0.25) (layer F.Cu) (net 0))
 (segment (start 154.2 90.5) (end 154.2 90.940381) (width 0.25) (layer F.Cu) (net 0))
 (segment (start 154.2 90.940381) (end 149.808668 95.331713) (width 0.25) (layer F.Cu) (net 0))
 (segment (start 155.8 91.02) (end 155.039619 91.02) (width 0.25) (layer F.Cu) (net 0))
 (segment (start 155.039619 91.02) (end 150.268287 95.791332) (width 0.25) (layer F.Cu) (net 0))
 (segment (start 155.8 93.56) (end 153.418858 93.56) (width 0.25) (layer F.Cu) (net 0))
 (segment (start 153.418858 93.56) (end 150.727907 96.250951) (width 0.25) (layer F.Cu) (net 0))
 (segment (start 148.889429 100.387526) (end 148.889429 100.389429) (width 0.25) (layer F.Cu) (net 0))
 (segment (start 148.889429 100.389429) (end 153.7 105.2) (width 0.25) (layer F.Cu) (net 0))
 (segment (start 153.7 105.2) (end 153.7 107) (width 0.25) (layer F.Cu) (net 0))
 (segment (start 153.7 107) (end 154.2 107.5) (width 0.25) (layer F.Cu) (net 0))
 (segment (start 154.2 107.5) (end 154.2 109.74) (width 0.25) (layer F.Cu) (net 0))
 (segment (start 154.2 109.74) (end 155.8 111.34) (width 0.25) (layer F.Cu) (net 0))
 (segment (start 155.8 108.8) (end 155.8 108.4) (width 0.25) (layer F.Cu) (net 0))
 (segment (start 155.8 108.4) (end 154.2 106.8) (width 0.25) (layer F.Cu) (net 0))
 (segment (start 154.2 106.8) (end 154.2 105) (width 0.25) (layer F.Cu) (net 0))
 (segment (start 154.2 105) (end 153.7 104.5) (width 0.25) (layer F.Cu) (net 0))
 (segment (start 153.7 104.5) (end 153.7 104.278858) (width 0.25) (layer F.Cu) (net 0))
 (segment (start 153.7 104.278858) (end 149.349049 99.927907) (width 0.25) (layer F.Cu) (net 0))
 (segment (start 155.8 106.26) (end 155.8 105.9) (width 0.25) (layer F.Cu) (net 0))
 (segment (start 155.8 105.9) (end 154.2 104.3) (width 0.25) (layer F.Cu) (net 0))
 (segment (start 154.2 104.3) (end 154.2 103.859619) (width 0.25) (layer F.Cu) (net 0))
 (segment (start 154.2 103.859619) (end 149.808668 99.468287) (width 0.25) (layer F.Cu) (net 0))
 (segment (start 155.8 103.72) (end 154.979619 103.72) (width 0.25) (layer F.Cu) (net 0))
 (segment (start 154.979619 103.72) (end 150.268287 99.008668) (width 0.25) (layer F.Cu) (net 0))
 (segment (start 155.8 101.18) (end 153.358858 101.18) (width 0.25) (layer F.Cu) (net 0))
 (segment (start 153.358858 101.18) (end 150.727907 98.549049) (width 0.25) (layer F.Cu) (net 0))
 (segment (start 155.8 96.1) (end 151.798097 96.1) (width 0.25) (layer F.Cu) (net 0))
 (segment (start 151.798097 96.1) (end 151.187526 96.710571) (width 0.25) (layer F.Cu) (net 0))
 (segment (start 155.8 98.64) (end 151.738097 98.64) (width 0.25) (layer F.Cu) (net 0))
 (segment (start 151.738097 98.64) (end 151.187526 98.089429) (width 0.25) (layer F.Cu) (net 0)))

